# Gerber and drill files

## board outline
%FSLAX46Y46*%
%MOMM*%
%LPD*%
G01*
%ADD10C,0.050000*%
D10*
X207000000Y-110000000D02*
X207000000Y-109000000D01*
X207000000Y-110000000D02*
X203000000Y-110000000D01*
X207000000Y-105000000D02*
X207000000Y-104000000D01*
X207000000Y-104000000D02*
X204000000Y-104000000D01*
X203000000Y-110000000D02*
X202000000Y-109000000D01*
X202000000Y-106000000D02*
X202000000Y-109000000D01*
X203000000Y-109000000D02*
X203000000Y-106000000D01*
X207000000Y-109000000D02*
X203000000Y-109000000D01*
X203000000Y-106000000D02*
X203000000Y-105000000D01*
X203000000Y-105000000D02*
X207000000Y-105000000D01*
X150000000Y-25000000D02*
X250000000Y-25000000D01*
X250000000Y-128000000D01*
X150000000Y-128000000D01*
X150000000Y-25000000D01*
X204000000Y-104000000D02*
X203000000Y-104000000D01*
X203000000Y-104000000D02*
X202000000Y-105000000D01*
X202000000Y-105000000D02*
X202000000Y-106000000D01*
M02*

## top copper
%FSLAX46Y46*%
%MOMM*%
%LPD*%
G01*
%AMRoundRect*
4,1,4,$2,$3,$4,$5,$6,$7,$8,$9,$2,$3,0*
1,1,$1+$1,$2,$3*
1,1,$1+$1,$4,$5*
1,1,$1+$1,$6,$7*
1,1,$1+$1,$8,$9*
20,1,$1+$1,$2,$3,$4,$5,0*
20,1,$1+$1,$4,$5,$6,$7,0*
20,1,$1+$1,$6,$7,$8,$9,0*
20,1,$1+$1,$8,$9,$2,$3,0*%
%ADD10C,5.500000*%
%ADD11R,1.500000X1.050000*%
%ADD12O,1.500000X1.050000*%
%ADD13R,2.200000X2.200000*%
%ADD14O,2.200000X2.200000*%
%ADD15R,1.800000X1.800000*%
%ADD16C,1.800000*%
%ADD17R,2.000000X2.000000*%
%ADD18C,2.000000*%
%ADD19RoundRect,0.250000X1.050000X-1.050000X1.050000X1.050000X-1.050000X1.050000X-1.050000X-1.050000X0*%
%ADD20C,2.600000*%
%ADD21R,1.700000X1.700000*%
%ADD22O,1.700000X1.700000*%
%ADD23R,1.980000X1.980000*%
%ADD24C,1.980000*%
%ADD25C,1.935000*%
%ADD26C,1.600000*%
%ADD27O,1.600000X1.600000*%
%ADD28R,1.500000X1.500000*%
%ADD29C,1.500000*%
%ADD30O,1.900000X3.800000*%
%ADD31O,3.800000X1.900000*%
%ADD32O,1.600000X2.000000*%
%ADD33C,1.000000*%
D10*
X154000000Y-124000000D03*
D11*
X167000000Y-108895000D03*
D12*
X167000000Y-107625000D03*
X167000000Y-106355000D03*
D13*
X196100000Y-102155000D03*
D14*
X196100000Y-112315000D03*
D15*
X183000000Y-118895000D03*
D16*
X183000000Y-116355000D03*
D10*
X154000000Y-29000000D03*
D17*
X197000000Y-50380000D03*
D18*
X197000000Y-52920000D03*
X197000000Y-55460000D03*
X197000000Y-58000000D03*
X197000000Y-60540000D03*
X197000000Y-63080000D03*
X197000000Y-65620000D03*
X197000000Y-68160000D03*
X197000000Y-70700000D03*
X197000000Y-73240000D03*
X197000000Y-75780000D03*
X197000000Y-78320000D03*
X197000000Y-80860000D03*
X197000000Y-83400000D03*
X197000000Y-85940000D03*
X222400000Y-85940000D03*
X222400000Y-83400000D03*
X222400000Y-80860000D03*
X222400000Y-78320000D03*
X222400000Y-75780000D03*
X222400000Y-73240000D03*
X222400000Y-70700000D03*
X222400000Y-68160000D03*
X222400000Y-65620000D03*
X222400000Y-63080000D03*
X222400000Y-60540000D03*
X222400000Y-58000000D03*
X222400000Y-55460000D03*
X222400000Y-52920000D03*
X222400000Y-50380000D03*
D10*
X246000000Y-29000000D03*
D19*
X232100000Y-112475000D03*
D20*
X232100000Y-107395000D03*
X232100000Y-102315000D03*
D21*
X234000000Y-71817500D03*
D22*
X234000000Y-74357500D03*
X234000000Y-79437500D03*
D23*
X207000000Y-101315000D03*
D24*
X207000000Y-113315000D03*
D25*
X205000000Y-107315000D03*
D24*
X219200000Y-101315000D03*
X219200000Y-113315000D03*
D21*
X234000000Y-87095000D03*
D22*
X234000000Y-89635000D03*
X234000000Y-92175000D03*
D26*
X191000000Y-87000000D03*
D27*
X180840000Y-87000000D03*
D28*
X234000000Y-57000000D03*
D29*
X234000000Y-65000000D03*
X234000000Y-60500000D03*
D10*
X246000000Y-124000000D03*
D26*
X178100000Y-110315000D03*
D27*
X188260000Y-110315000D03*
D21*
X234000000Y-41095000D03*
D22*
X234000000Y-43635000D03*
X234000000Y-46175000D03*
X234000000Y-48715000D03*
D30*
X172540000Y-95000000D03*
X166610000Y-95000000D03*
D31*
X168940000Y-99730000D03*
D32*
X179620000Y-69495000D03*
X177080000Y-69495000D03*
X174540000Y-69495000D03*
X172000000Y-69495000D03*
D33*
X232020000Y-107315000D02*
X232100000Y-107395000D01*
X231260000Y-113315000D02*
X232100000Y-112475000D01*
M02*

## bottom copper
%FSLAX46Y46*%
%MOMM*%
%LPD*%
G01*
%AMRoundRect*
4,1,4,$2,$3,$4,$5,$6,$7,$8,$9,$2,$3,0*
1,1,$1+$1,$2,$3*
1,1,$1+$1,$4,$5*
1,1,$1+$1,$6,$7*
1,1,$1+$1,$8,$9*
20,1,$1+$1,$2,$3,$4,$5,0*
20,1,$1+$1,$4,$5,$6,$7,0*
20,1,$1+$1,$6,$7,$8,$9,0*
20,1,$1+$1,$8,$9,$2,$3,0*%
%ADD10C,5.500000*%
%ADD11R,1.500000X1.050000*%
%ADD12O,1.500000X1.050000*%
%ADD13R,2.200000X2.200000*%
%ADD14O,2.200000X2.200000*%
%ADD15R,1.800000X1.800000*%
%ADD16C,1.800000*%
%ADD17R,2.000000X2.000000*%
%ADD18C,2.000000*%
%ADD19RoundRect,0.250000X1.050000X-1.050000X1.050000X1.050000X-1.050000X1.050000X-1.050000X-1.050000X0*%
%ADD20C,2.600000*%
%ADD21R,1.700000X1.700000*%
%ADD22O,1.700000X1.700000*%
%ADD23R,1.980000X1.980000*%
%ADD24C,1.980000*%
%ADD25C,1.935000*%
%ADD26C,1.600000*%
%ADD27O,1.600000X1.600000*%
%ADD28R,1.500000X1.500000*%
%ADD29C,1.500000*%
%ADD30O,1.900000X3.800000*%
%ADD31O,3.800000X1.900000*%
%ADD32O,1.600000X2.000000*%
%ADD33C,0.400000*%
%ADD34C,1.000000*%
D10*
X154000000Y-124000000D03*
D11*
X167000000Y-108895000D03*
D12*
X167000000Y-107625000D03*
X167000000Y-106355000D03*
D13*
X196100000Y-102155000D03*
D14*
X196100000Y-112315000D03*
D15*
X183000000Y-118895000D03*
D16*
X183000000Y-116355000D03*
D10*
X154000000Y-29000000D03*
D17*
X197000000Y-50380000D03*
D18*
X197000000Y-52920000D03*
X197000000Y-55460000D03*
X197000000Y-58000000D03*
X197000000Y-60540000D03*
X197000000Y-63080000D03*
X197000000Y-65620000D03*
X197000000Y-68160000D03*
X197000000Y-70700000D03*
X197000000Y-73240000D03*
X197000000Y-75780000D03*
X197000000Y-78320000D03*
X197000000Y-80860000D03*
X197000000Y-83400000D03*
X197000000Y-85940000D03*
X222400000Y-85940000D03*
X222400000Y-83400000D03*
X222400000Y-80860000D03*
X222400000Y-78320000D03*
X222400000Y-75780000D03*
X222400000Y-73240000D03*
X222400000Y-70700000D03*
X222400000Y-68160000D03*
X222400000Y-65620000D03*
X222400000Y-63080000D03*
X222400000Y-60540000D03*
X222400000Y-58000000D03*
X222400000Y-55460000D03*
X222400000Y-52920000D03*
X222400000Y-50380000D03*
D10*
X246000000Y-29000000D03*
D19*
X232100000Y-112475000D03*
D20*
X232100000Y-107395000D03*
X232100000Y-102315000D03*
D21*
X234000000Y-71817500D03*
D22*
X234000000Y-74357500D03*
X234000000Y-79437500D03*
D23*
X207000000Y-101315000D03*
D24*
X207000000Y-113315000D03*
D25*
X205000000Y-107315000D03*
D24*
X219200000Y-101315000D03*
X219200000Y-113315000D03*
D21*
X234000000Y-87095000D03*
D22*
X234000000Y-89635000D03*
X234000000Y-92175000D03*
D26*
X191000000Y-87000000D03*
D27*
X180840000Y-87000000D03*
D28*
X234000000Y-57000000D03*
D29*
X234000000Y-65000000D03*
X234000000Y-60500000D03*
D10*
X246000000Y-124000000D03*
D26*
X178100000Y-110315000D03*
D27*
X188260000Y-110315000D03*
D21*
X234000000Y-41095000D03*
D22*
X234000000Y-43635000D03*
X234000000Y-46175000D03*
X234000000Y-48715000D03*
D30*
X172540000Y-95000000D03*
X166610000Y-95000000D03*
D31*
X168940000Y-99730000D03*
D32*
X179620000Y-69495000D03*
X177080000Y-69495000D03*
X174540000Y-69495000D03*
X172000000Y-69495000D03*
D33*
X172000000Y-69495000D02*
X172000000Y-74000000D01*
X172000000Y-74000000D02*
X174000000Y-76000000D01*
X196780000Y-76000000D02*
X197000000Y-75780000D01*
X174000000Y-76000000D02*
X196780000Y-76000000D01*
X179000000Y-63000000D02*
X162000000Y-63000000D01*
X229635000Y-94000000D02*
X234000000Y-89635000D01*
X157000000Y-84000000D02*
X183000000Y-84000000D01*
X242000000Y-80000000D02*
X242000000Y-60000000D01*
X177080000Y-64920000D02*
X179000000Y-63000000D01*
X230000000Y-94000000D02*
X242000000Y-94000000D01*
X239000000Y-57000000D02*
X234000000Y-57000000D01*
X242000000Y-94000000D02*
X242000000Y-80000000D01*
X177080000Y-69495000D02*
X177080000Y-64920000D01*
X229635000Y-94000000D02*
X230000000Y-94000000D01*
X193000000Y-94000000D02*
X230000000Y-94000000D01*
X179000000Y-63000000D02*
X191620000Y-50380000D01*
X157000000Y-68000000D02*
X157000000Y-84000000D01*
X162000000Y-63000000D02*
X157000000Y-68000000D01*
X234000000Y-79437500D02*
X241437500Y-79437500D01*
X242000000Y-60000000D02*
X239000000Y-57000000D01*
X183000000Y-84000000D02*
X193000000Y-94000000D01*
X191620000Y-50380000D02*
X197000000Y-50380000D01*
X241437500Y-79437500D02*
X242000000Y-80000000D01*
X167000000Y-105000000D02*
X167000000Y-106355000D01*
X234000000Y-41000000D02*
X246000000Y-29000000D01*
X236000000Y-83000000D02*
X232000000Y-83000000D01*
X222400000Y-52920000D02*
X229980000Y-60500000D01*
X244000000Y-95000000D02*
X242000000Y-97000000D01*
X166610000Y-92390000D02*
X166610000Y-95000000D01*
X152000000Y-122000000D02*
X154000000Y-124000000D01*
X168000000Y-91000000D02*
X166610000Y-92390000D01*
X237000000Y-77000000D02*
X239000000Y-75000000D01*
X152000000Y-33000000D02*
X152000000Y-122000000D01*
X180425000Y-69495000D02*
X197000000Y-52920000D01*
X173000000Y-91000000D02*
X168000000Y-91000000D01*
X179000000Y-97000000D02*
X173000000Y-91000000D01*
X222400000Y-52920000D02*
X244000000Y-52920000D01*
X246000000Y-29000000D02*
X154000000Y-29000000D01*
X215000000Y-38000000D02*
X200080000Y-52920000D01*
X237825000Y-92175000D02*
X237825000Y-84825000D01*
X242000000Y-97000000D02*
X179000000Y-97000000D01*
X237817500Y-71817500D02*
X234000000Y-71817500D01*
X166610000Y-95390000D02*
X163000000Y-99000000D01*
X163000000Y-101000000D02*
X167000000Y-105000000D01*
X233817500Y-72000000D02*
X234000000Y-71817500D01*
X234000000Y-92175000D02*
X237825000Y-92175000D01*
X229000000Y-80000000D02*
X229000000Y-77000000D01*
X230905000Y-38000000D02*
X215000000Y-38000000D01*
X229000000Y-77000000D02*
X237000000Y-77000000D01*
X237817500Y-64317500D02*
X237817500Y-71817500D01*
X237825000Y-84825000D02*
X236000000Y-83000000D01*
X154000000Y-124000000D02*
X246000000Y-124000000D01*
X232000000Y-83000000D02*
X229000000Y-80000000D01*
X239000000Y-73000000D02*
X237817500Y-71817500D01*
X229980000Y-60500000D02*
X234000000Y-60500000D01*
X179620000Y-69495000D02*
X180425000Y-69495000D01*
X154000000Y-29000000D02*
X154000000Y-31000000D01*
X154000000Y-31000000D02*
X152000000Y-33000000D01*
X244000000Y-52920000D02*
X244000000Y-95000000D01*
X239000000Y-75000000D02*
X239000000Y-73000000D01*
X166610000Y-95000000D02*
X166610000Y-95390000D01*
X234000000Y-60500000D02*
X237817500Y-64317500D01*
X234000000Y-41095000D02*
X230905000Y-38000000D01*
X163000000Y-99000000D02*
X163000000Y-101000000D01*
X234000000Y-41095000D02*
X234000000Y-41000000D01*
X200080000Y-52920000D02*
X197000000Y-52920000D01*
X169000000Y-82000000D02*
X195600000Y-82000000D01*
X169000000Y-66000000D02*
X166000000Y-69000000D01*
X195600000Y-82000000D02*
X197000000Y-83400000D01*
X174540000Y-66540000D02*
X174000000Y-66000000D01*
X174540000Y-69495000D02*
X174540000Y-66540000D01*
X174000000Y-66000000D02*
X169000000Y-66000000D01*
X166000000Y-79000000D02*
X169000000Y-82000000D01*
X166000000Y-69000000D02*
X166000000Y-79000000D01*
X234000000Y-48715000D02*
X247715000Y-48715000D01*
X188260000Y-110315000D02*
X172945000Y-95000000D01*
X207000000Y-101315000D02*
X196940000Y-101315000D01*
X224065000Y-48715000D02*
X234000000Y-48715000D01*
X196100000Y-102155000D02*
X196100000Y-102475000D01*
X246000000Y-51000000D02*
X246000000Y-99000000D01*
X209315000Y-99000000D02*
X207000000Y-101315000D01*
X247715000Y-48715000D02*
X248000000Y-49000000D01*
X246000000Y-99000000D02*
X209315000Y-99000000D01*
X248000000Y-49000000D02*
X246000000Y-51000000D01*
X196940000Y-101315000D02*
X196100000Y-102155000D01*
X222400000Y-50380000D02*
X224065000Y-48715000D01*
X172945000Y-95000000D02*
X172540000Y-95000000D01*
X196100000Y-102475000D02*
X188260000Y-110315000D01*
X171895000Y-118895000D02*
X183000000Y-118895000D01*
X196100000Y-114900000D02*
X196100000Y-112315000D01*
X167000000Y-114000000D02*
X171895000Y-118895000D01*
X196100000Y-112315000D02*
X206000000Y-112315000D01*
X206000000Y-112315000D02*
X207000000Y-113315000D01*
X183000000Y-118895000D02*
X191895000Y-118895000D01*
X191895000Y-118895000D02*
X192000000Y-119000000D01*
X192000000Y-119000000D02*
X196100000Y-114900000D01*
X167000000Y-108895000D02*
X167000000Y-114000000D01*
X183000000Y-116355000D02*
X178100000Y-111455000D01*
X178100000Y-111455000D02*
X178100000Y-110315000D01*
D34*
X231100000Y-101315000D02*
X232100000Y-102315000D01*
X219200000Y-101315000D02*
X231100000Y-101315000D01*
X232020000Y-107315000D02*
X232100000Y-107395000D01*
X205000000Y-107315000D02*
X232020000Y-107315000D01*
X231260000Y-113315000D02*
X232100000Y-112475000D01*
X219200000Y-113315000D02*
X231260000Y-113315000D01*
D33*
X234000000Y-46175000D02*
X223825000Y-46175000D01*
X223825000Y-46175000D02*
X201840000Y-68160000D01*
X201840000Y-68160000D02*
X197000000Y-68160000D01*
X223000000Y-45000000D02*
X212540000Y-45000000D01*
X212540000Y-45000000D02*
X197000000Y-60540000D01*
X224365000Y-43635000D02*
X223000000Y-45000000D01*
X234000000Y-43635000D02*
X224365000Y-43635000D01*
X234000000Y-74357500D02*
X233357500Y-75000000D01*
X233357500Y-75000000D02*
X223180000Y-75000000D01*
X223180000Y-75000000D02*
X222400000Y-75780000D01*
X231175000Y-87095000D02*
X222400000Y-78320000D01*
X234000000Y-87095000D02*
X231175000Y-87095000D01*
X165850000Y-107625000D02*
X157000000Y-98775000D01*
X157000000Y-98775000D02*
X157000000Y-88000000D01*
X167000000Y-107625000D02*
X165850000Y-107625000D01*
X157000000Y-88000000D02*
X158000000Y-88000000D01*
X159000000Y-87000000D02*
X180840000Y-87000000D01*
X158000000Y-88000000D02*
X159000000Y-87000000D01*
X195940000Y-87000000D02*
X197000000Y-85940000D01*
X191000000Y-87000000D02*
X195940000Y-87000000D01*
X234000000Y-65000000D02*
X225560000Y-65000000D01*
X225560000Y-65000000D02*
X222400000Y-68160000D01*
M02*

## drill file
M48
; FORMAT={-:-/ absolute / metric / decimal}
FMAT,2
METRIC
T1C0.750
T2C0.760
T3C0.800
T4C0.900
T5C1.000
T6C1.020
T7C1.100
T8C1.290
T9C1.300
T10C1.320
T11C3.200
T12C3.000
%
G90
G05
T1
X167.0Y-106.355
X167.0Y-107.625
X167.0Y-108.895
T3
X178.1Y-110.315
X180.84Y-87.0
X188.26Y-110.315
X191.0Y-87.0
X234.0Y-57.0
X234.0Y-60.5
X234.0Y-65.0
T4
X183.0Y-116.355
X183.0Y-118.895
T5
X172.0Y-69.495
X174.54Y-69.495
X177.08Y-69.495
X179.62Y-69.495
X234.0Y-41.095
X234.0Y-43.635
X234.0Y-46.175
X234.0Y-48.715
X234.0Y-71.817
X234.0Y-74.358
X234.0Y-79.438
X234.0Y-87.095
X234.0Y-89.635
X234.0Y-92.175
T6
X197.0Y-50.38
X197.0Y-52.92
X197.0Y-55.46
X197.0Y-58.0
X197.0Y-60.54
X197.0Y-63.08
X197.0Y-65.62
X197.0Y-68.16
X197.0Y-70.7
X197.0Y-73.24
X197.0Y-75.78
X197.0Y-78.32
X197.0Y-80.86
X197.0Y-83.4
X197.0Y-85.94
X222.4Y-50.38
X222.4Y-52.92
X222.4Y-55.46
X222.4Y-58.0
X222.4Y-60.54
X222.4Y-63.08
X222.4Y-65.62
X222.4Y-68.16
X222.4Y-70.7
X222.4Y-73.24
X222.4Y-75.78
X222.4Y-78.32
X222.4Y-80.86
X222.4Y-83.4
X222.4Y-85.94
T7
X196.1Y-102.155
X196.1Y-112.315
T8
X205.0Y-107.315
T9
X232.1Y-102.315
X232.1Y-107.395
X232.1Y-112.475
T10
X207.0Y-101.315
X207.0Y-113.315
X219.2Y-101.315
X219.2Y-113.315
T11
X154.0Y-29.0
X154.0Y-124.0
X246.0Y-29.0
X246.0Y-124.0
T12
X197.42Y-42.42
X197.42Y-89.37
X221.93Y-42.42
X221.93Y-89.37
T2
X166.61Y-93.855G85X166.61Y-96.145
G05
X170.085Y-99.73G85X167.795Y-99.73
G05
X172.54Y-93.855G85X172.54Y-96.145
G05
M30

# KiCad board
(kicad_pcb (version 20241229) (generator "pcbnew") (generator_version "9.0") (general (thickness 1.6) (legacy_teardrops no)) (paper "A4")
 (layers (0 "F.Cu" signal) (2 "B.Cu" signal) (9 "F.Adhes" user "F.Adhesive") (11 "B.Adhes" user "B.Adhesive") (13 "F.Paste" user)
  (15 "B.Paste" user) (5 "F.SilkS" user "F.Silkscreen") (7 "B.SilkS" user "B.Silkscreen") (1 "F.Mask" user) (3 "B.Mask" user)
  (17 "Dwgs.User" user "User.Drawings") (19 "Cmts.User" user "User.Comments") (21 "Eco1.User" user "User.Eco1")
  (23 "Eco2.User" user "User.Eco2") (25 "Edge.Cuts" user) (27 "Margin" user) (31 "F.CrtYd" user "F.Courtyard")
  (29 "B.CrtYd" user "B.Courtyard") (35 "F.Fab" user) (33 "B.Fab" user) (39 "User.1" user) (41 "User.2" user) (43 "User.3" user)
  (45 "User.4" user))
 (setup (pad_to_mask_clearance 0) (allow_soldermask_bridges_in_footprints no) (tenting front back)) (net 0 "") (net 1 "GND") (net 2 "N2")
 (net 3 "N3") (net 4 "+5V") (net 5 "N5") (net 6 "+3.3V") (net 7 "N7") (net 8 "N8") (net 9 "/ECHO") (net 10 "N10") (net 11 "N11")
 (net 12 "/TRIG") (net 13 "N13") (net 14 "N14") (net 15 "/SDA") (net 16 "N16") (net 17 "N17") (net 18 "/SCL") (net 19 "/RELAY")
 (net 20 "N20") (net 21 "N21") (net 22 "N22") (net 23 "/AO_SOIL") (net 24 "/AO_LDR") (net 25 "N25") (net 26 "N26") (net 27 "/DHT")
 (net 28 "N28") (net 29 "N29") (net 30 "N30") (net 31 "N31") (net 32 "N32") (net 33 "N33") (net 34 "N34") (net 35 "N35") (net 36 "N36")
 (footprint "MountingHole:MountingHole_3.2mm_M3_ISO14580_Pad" (layer "F.Cu") (at 154 124)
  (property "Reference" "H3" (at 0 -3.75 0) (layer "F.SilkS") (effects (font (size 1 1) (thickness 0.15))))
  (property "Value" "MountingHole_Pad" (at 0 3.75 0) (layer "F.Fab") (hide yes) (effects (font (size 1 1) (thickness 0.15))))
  (pad "1" thru_hole circle (at 0 0) (size 5.5 5.5) (drill 3.2) (layers "*.Cu" "*.Mask") (remove_unused_layers no) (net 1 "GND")))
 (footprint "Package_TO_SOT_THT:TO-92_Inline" (layer "F.Cu") (at 167 108.895 90)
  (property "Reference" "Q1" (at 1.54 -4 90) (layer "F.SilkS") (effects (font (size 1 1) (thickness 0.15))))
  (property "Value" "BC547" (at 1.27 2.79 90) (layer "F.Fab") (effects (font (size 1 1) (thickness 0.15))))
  (pad "1" thru_hole rect (at 0 0 90) (size 1.05 1.5) (drill 0.75) (layers "*.Cu" "*.Mask") (remove_unused_layers no) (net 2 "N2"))
  (pad "2" thru_hole oval (at 1.27 0 90) (size 1.05 1.5) (drill 0.75) (layers "*.Cu" "*.Mask") (remove_unused_layers no) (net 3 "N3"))
  (pad "3" thru_hole oval (at 2.54 0 90) (size 1.05 1.5) (drill 0.75) (layers "*.Cu" "*.Mask") (remove_unused_layers no) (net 1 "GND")))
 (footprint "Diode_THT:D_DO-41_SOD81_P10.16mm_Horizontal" (layer "F.Cu") (at 196.1 102.155 -90)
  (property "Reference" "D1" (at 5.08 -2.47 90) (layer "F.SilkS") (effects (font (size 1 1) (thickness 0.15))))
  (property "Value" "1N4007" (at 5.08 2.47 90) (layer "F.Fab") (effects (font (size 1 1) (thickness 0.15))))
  (pad "1" thru_hole rect (at 0 0 270) (size 2.2 2.2) (drill 1.1) (layers "*.Cu" "*.Mask") (remove_unused_layers no) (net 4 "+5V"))
  (pad "2" thru_hole oval (at 10.16 0 270) (size 2.2 2.2) (drill 1.1) (layers "*.Cu" "*.Mask") (remove_unused_layers no) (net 2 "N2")))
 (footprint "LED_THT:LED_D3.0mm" (layer "F.Cu") (at 183 118.895 90)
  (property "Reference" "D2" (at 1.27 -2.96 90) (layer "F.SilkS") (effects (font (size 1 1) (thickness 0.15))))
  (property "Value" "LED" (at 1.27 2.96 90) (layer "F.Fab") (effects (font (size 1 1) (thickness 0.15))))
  (pad "1" thru_hole rect (at 0 0 90) (size 1.8 1.8) (drill 0.9) (layers "*.Cu" "*.Mask") (remove_unused_layers no) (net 2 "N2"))
  (pad "2" thru_hole circle (at 2.54 0 90) (size 1.8 1.8) (drill 0.9) (layers "*.Cu" "*.Mask") (remove_unused_layers no) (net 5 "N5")))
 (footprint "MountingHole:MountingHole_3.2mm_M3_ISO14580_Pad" (layer "F.Cu") (at 154 29)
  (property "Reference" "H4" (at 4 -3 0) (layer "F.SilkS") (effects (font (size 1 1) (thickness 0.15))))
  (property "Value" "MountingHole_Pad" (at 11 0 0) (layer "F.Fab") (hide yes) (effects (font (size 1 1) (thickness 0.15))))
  (pad "1" thru_hole circle (at 0 0) (size 5.5 5.5) (drill 3.2) (layers "*.Cu" "*.Mask") (remove_unused_layers no) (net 1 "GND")))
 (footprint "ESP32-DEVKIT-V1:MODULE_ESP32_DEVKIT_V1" (layer "F.Cu") (at 209.7 65.895)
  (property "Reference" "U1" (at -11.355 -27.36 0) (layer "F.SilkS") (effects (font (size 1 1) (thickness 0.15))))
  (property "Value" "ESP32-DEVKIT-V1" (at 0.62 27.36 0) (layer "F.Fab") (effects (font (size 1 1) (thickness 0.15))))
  (pad "" np_thru_hole circle (at -12.28 -23.475) (size 3 3) (drill 3) (layers "*.Cu" "*.Mask"))
  (pad "" np_thru_hole circle (at -12.28 23.475) (size 3 3) (drill 3) (layers "*.Cu" "*.Mask"))
  (pad "" np_thru_hole circle (at 12.23 -23.475) (size 3 3) (drill 3) (layers "*.Cu" "*.Mask"))
  (pad "" np_thru_hole circle (at 12.23 23.475) (size 3 3) (drill 3) (layers "*.Cu" "*.Mask"))
  (pad "1" thru_hole rect (at -12.7 -15.515) (size 2 2) (drill 1.02) (layers "*.Cu" "*.Mask") (remove_unused_layers no) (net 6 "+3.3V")
   (solder_mask_margin 0.102))
  (pad "2" thru_hole circle (at -12.7 -12.975) (size 2 2) (drill 1.02) (layers "*.Cu" "*.Mask") (remove_unused_layers no) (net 1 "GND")
   (solder_mask_margin 0.102))
  (pad "3" thru_hole circle (at -12.7 -10.435) (size 2 2) (drill 1.02) (layers "*.Cu" "*.Mask") (remove_unused_layers no) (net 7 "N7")
   (solder_mask_margin 0.102))
  (pad "4" thru_hole circle (at -12.7 -7.895) (size 2 2) (drill 1.02) (layers "*.Cu" "*.Mask") (remove_unused_layers no) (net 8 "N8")
   (solder_mask_margin 0.102))
  (pad "5" thru_hole circle (at -12.7 -5.355) (size 2 2) (drill 1.02) (layers "*.Cu" "*.Mask") (remove_unused_layers no) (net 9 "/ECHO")
   (solder_mask_margin 0.102))
  (pad "6" thru_hole circle (at -12.7 -2.815) (size 2 2) (drill 1.02) (layers "*.Cu" "*.Mask") (remove_unused_layers no) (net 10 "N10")
   (solder_mask_margin 0.102))
  (pad "7" thru_hole circle (at -12.7 -0.275) (size 2 2) (drill 1.02) (layers "*.Cu" "*.Mask") (remove_unused_layers no) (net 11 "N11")
   (solder_mask_margin 0.102))
  (pad "8" thru_hole circle (at -12.7 2.265) (size 2 2) (drill 1.02) (layers "*.Cu" "*.Mask") (remove_unused_layers no) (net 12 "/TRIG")
   (solder_mask_margin 0.102))
  (pad "9" thru_hole circle (at -12.7 4.805) (size 2 2) (drill 1.02) (layers "*.Cu" "*.Mask") (remove_unused_layers no) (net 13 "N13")
   (solder_mask_margin 0.102))
  (pad "10" thru_hole circle (at -12.7 7.345) (size 2 2) (drill 1.02) (layers "*.Cu" "*.Mask") (remove_unused_layers no) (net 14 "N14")
   (solder_mask_margin 0.102))
  (pad "11" thru_hole circle (at -12.7 9.885) (size 2 2) (drill 1.02) (layers "*.Cu" "*.Mask") (remove_unused_layers no) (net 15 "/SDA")
   (solder_mask_margin 0.102))
  (pad "12" thru_hole circle (at -12.7 12.425) (size 2 2) (drill 1.02) (layers "*.Cu" "*.Mask") (remove_unused_layers no) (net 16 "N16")
   (solder_mask_margin 0.102))
  (pad "13" thru_hole circle (at -12.7 14.965) (size 2 2) (drill 1.02) (layers "*.Cu" "*.Mask") (remove_unused_layers no) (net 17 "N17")
   (solder_mask_margin 0.102))
  (pad "14" thru_hole circle (at -12.7 17.505) (size 2 2) (drill 1.02) (layers "*.Cu" "*.Mask") (remove_unused_layers no) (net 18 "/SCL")
   (solder_mask_margin 0.102))
  (pad "15" thru_hole circle (at -12.7 20.045) (size 2 2) (drill 1.02) (layers "*.Cu" "*.Mask") (remove_unused_layers no) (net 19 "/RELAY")
   (solder_mask_margin 0.102))
  (pad "16" thru_hole circle (at 12.7 20.045) (size 2 2) (drill 1.02) (layers "*.Cu" "*.Mask") (remove_unused_layers no) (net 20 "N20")
   (solder_mask_margin 0.102))
  (pad "17" thru_hole circle (at 12.7 17.505) (size 2 2) (drill 1.02) (layers "*.Cu" "*.Mask") (remove_unused_layers no) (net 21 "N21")
   (solder_mask_margin 0.102))
  (pad "18" thru_hole circle (at 12.7 14.965) (size 2 2) (drill 1.02) (layers "*.Cu" "*.Mask") (remove_unused_layers no) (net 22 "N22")
   (solder_mask_margin 0.102))
  (pad "19" thru_hole circle (at 12.7 12.425) (size 2 2) (drill 1.02) (layers "*.Cu" "*.Mask") (remove_unused_layers no) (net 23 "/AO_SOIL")
   (solder_mask_margin 0.102))
  (pad "20" thru_hole circle (at 12.7 9.885) (size 2 2) (drill 1.02) (layers "*.Cu" "*.Mask") (remove_unused_layers no) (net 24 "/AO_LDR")
   (solder_mask_margin 0.102))
  (pad "21" thru_hole circle (at 12.7 7.345) (size 2 2) (drill 1.02) (layers "*.Cu" "*.Mask") (remove_unused_layers no) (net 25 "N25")
   (solder_mask_margin 0.102))
  (pad "22" thru_hole circle (at 12.7 4.805) (size 2 2) (drill 1.02) (layers "*.Cu" "*.Mask") (remove_unused_layers no) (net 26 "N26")
   (solder_mask_margin 0.102))
  (pad "23" thru_hole circle (at 12.7 2.265) (size 2 2) (drill 1.02) (layers "*.Cu" "*.Mask") (remove_unused_layers no) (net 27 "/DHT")
   (solder_mask_margin 0.102))
  (pad "24" thru_hole circle (at 12.7 -0.275) (size 2 2) (drill 1.02) (layers "*.Cu" "*.Mask") (remove_unused_layers no) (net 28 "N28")
   (solder_mask_margin 0.102))
  (pad "25" thru_hole circle (at 12.7 -2.815) (size 2 2) (drill 1.02) (layers "*.Cu" "*.Mask") (remove_unused_layers no) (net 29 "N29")
   (solder_mask_margin 0.102))
  (pad "26" thru_hole circle (at 12.7 -5.355) (size 2 2) (drill 1.02) (layers "*.Cu" "*.Mask") (remove_unused_layers no) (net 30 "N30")
   (solder_mask_margin 0.102))
  (pad "27" thru_hole circle (at 12.7 -7.895) (size 2 2) (drill 1.02) (layers "*.Cu" "*.Mask") (remove_unused_layers no) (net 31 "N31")
   (solder_mask_margin 0.102))
  (pad "28" thru_hole circle (at 12.7 -10.435) (size 2 2) (drill 1.02) (layers "*.Cu" "*.Mask") (remove_unused_layers no) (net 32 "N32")
   (solder_mask_margin 0.102))
  (pad "29" thru_hole circle (at 12.7 -12.975) (size 2 2) (drill 1.02) (layers "*.Cu" "*.Mask") (remove_unused_layers no) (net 1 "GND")
   (solder_mask_margin 0.102))
  (pad "30" thru_hole circle (at 12.7 -15.515) (size 2 2) (drill 1.02) (layers "*.Cu" "*.Mask") (remove_unused_layers no) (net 4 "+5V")
   (solder_mask_margin 0.102))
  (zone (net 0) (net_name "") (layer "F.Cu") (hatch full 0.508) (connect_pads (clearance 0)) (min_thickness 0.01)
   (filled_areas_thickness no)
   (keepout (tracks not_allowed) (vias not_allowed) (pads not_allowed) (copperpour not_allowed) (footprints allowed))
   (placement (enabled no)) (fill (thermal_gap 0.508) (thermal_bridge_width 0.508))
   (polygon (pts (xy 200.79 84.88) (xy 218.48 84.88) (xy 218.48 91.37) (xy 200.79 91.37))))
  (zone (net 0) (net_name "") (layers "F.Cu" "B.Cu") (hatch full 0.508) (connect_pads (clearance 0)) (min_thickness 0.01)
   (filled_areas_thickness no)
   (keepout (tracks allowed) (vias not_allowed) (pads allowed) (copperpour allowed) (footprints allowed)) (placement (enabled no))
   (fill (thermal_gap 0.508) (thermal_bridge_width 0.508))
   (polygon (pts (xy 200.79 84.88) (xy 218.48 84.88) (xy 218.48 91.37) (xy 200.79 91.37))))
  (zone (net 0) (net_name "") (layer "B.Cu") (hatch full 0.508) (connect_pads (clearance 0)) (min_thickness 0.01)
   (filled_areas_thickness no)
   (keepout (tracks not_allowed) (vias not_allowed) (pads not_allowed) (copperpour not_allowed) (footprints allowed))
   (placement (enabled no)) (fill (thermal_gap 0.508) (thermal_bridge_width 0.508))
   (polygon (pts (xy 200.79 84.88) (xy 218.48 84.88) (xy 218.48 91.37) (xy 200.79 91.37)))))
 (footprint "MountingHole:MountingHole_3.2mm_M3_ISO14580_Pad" (layer "F.Cu") (at 246 29)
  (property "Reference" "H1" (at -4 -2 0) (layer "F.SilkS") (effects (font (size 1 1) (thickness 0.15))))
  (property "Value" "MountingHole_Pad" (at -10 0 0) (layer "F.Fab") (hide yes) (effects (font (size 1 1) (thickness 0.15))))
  (pad "1" thru_hole circle (at 0 0) (size 5.5 5.5) (drill 3.2) (layers "*.Cu" "*.Mask") (remove_unused_layers no) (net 1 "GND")))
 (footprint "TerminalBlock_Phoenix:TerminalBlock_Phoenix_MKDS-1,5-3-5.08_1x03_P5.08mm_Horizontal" (layer "F.Cu") (at 232.1 112.475 90)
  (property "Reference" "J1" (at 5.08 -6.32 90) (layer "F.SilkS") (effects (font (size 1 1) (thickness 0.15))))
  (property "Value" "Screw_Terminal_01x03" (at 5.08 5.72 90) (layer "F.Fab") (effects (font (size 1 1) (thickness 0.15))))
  (pad "1" thru_hole roundrect (at 0 0 90) (size 2.6 2.6) (drill 1.3) (layers "*.Cu" "*.Mask") (remove_unused_layers no)
   (roundrect_rratio 0.096154) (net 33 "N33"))
  (pad "2" thru_hole circle (at 5.08 0 90) (size 2.6 2.6) (drill 1.3) (layers "*.Cu" "*.Mask") (remove_unused_layers no) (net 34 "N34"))
  (pad "3" thru_hole circle (at 10.16 0 90) (size 2.6 2.6) (drill 1.3) (layers "*.Cu" "*.Mask") (remove_unused_layers no) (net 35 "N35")))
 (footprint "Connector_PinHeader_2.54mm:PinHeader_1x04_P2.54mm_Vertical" (layer "F.Cu") (at 234 71.8175)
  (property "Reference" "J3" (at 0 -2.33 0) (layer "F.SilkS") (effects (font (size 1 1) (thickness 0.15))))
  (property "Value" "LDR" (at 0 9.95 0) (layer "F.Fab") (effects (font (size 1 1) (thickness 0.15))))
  (pad "1" thru_hole rect (at 0 0) (size 1.7 1.7) (drill 1) (layers "*.Cu" "*.Mask") (remove_unused_layers no) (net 1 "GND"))
  (pad "2" thru_hole oval (at 0 2.54) (size 1.7 1.7) (drill 1) (layers "*.Cu" "*.Mask") (remove_unused_layers no) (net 24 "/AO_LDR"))
  (pad "4" thru_hole oval (at 0 7.62) (size 1.7 1.7) (drill 1) (layers "*.Cu" "*.Mask") (remove_unused_layers no) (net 6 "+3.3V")))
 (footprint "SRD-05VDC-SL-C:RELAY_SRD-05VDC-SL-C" (layer "F.Cu") (at 213.1 107.315)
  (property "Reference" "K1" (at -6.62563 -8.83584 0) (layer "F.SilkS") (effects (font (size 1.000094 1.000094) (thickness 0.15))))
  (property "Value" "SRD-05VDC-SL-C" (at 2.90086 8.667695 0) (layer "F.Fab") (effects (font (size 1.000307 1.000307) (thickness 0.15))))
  (pad "A1" thru_hole rect (at -6.1 -6) (size 1.98 1.98) (drill 1.32) (layers "*.Cu" "*.Mask") (remove_unused_layers no) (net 4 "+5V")
   (solder_mask_margin 0.102))
  (pad "A2" thru_hole circle (at -6.1 6) (size 1.98 1.98) (drill 1.32) (layers "*.Cu" "*.Mask") (remove_unused_layers no) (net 2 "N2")
   (solder_mask_margin 0.102))
  (pad "COM" thru_hole circle (at -8.1 0) (size 1.935 1.935) (drill 1.29) (layers "*.Cu" "*.Mask") (remove_unused_layers no) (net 34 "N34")
   (solder_mask_margin 0.102))
  (pad "NC" thru_hole circle (at 6.1 -6) (size 1.98 1.98) (drill 1.32) (layers "*.Cu" "*.Mask") (remove_unused_layers no) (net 35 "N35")
   (solder_mask_margin 0.102))
  (pad "NO" thru_hole circle (at 6.1 6) (size 1.98 1.98) (drill 1.32) (layers "*.Cu" "*.Mask") (remove_unused_layers no) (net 33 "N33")
   (solder_mask_margin 0.102)))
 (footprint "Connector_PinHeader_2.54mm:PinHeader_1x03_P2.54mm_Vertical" (layer "F.Cu") (at 234 87.095)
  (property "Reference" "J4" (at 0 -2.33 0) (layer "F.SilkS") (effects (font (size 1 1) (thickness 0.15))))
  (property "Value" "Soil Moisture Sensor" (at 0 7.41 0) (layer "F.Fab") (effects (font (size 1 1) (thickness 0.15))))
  (pad "1" thru_hole rect (at 0 0) (size 1.7 1.7) (drill 1) (layers "*.Cu" "*.Mask") (remove_unused_layers no) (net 23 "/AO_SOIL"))
  (pad "2" thru_hole oval (at 0 2.54) (size 1.7 1.7) (drill 1) (layers "*.Cu" "*.Mask") (remove_unused_layers no) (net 6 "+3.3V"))
  (pad "3" thru_hole oval (at 0 5.08) (size 1.7 1.7) (drill 1) (layers "*.Cu" "*.Mask") (remove_unused_layers no) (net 1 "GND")))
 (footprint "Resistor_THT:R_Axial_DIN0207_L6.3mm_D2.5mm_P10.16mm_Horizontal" (layer "F.Cu") (at 191 87 180)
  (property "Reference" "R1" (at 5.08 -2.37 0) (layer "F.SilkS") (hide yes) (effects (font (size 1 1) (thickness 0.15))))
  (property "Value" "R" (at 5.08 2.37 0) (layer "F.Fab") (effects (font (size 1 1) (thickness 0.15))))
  (pad "1" thru_hole circle (at 0 0 180) (size 1.6 1.6) (drill 0.8) (layers "*.Cu" "*.Mask") (remove_unused_layers no) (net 19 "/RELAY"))
  (pad "2" thru_hole oval (at 10.16 0 180) (size 1.6 1.6) (drill 0.8) (layers "*.Cu" "*.Mask") (remove_unused_layers no) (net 3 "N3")))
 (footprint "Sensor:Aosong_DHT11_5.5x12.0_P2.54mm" (layer "F.Cu") (at 234 57)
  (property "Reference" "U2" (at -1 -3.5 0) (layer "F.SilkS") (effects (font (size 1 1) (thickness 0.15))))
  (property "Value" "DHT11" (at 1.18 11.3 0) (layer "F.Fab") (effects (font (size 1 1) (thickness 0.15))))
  (pad "1" thru_hole rect (at 0 0) (size 1.5 1.5) (drill 0.8) (layers "*.Cu" "*.Mask") (remove_unused_layers no) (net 6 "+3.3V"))
  (pad "2" thru_hole circle (at 0 8) (size 1.5 1.5) (drill 0.8) (layers "*.Cu" "*.Mask") (remove_unused_layers no) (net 27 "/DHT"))
  (pad "4" thru_hole circle (at 0 3.5) (size 1.5 1.5) (drill 0.8) (layers "*.Cu" "*.Mask") (remove_unused_layers no) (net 1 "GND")))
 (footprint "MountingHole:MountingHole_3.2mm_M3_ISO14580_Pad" (layer "F.Cu") (at 246 124)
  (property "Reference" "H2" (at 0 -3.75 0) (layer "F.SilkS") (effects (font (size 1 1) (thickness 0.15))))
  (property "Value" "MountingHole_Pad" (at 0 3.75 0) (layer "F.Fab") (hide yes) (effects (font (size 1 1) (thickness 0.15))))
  (pad "1" thru_hole circle (at 0 0) (size 5.5 5.5) (drill 3.2) (layers "*.Cu" "*.Mask") (remove_unused_layers no) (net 1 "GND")))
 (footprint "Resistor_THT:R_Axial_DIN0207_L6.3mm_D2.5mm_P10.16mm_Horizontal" (layer "F.Cu") (at 178.1 110.315)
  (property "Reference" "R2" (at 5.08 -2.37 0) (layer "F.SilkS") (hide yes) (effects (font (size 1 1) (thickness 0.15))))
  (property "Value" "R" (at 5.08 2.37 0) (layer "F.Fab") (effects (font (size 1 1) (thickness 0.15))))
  (pad "1" thru_hole circle (at 0 0) (size 1.6 1.6) (drill 0.8) (layers "*.Cu" "*.Mask") (remove_unused_layers no) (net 5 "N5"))
  (pad "2" thru_hole oval (at 10.16 0) (size 1.6 1.6) (drill 0.8) (layers "*.Cu" "*.Mask") (remove_unused_layers no) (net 4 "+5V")))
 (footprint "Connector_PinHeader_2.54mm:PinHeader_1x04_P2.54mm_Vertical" (layer "F.Cu") (at 234 41.095)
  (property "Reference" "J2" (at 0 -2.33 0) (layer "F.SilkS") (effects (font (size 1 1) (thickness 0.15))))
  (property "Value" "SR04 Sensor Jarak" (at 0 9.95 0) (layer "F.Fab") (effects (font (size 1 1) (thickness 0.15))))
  (pad "1" thru_hole rect (at 0 0) (size 1.7 1.7) (drill 1) (layers "*.Cu" "*.Mask") (remove_unused_layers no) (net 1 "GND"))
  (pad "2" thru_hole oval (at 0 2.54) (size 1.7 1.7) (drill 1) (layers "*.Cu" "*.Mask") (remove_unused_layers no) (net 9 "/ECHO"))
  (pad "3" thru_hole oval (at 0 5.08) (size 1.7 1.7) (drill 1) (layers "*.Cu" "*.Mask") (remove_unused_layers no) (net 12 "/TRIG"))
  (pad "4" thru_hole oval (at 0 7.62) (size 1.7 1.7) (drill 1) (layers "*.Cu" "*.Mask") (remove_unused_layers no) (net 4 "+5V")))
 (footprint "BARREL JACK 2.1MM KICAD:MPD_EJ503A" (layer "F.Cu") (at 166 95 -90)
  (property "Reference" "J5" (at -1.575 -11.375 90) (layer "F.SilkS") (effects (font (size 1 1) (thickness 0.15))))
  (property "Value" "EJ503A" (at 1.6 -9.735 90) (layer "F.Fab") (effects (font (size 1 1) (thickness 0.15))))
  (pad "1" thru_hole oval (at 0 -6.54 270) (size 3.8 1.9) (drill oval 3.05 0.76) (layers "*.Cu" "*.Mask") (remove_unused_layers no)
   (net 4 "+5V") (solder_mask_margin 0.102))
  (pad "2" thru_hole oval (at 0 -0.61 270) (size 3.8 1.9) (drill oval 3.05 0.76) (layers "*.Cu" "*.Mask") (remove_unused_layers no)
   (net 1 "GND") (solder_mask_margin 0.102))
  (pad "3" thru_hole oval (at 4.73 -2.94 270) (size 1.9 3.8) (drill oval 0.76 3.05) (layers "*.Cu" "*.Mask") (remove_unused_layers no)
   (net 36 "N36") (solder_mask_margin 0.102)))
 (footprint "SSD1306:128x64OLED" (layer "F.Cu") (at 176 58.895 180)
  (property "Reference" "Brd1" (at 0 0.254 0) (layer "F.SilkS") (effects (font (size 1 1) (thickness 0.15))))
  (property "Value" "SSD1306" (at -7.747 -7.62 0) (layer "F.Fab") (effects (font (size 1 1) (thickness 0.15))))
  (pad "1" thru_hole oval (at -3.62 -10.6 270) (size 2 1.6) (drill 1) (layers "*.Cu" "*.Mask") (remove_unused_layers no) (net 1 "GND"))
  (pad "2" thru_hole oval (at -1.08 -10.6 270) (size 2 1.6) (drill 1) (layers "*.Cu" "*.Mask") (remove_unused_layers no) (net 6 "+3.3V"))
  (pad "3" thru_hole oval (at 1.46 -10.6 270) (size 2 1.6) (drill 1) (layers "*.Cu" "*.Mask") (remove_unused_layers no) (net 18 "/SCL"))
  (pad "4" thru_hole oval (at 4 -10.6 270) (size 2 1.6) (drill 1) (layers "*.Cu" "*.Mask") (remove_unused_layers no) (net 15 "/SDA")))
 (gr_line (start 207 110) (end 207 109) (stroke (width 0.05) (type default)) (layer "Edge.Cuts"))
 (gr_line (start 207 110) (end 203 110) (stroke (width 0.05) (type default)) (layer "Edge.Cuts"))
 (gr_line (start 207 105) (end 207 104) (stroke (width 0.05) (type default)) (layer "Edge.Cuts"))
 (gr_line (start 207 104) (end 204 104) (stroke (width 0.05) (type default)) (layer "Edge.Cuts"))
 (gr_line (start 203 110) (end 202 109) (stroke (width 0.05) (type default)) (layer "Edge.Cuts"))
 (gr_line (start 202 106) (end 202 109) (stroke (width 0.05) (type default)) (layer "Edge.Cuts"))
 (gr_line (start 203 109) (end 203 106) (stroke (width 0.05) (type default)) (layer "Edge.Cuts"))
 (gr_line (start 207 109) (end 203 109) (stroke (width 0.05) (type default)) (layer "Edge.Cuts"))
 (gr_line (start 203 106) (end 203 105) (stroke (width 0.05) (type default)) (layer "Edge.Cuts"))
 (gr_line (start 203 105) (end 207 105) (stroke (width 0.05) (type default)) (layer "Edge.Cuts"))
 (gr_rect (start 150 25) (end 250 128) (stroke (width 0.05) (type default)) (fill no) (layer "Edge.Cuts"))
 (gr_line (start 204 104) (end 203 104) (stroke (width 0.05) (type default)) (layer "Edge.Cuts"))
 (gr_line (start 203 104) (end 202 105) (stroke (width 0.05) (type default)) (layer "Edge.Cuts"))
 (gr_line (start 202 105) (end 202 106) (stroke (width 0.05) (type default)) (layer "Edge.Cuts"))
 (segment (start 172 69.495) (end 172 74) (width 0.4) (layer "B.Cu") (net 15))
 (segment (start 172 74) (end 174 76) (width 0.4) (layer "B.Cu") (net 15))
 (segment (start 196.78 76) (end 197 75.78) (width 0.4) (layer "B.Cu") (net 15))
 (segment (start 174 76) (end 196.78 76) (width 0.4) (layer "B.Cu") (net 15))
 (segment (start 179 63) (end 162 63) (width 0.4) (layer "B.Cu") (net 6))
 (segment (start 229.635 94) (end 234 89.635) (width 0.4) (layer "B.Cu") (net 6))
 (segment (start 157 84) (end 183 84) (width 0.4) (layer "B.Cu") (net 6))
 (segment (start 242 80) (end 242 60) (width 0.4) (layer "B.Cu") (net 6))
 (segment (start 177.08 64.92) (end 179 63) (width 0.4) (layer "B.Cu") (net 6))
 (segment (start 230 94) (end 242 94) (width 0.4) (layer "B.Cu") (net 6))
 (segment (start 239 57) (end 234 57) (width 0.4) (layer "B.Cu") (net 6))
 (segment (start 242 94) (end 242 80) (width 0.4) (layer "B.Cu") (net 6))
 (segment (start 177.08 69.495) (end 177.08 64.92) (width 0.4) (layer "B.Cu") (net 6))
 (segment (start 229.635 94) (end 230 94) (width 0.4) (layer "B.Cu") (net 6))
 (segment (start 193 94) (end 230 94) (width 0.4) (layer "B.Cu") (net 6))
 (segment (start 179 63) (end 191.62 50.38) (width 0.4) (layer "B.Cu") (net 6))
 (segment (start 157 68) (end 157 84) (width 0.4) (layer "B.Cu") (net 6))
 (segment (start 162 63) (end 157 68) (width 0.4) (layer "B.Cu") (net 6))
 (segment (start 234 79.4375) (end 241.4375 79.4375) (width 0.4) (layer "B.Cu") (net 6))
 (segment (start 242 60) (end 239 57) (width 0.4) (layer "B.Cu") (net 6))
 (segment (start 183 84) (end 193 94) (width 0.4) (layer "B.Cu") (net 6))
 (segment (start 191.62 50.38) (end 197 50.38) (width 0.4) (layer "B.Cu") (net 6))
 (segment (start 241.4375 79.4375) (end 242 80) (width 0.4) (layer "B.Cu") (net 6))
 (segment (start 167 105) (end 167 106.355) (width 0.4) (layer "B.Cu") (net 1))
 (segment (start 234 41) (end 246 29) (width 0.4) (layer "B.Cu") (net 1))
 (segment (start 236 83) (end 232 83) (width 0.4) (layer "B.Cu") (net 1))
 (segment (start 222.4 52.92) (end 229.98 60.5) (width 0.4) (layer "B.Cu") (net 1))
 (segment (start 244 95) (end 242 97) (width 0.4) (layer "B.Cu") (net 1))
 (segment (start 166.61 92.39) (end 166.61 95) (width 0.4) (layer "B.Cu") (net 1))
 (segment (start 152 122) (end 154 124) (width 0.4) (layer "B.Cu") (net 1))
 (segment (start 168 91) (end 166.61 92.39) (width 0.4) (layer "B.Cu") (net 1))
 (segment (start 237 77) (end 239 75) (width 0.4) (layer "B.Cu") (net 1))
 (segment (start 152 33) (end 152 122) (width 0.4) (layer "B.Cu") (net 1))
 (segment (start 180.425 69.495) (end 197 52.92) (width 0.4) (layer "B.Cu") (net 1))
 (segment (start 173 91) (end 168 91) (width 0.4) (layer "B.Cu") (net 1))
 (segment (start 179 97) (end 173 91) (width 0.4) (layer "B.Cu") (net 1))
 (segment (start 222.4 52.92) (end 244 52.92) (width 0.4) (layer "B.Cu") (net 1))
 (segment (start 246 29) (end 154 29) (width 0.4) (layer "B.Cu") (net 1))
 (segment (start 215 38) (end 200.08 52.92) (width 0.4) (layer "B.Cu") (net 1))
 (segment (start 237.825 92.175) (end 237.825 84.825) (width 0.4) (layer "B.Cu") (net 1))
 (segment (start 242 97) (end 179 97) (width 0.4) (layer "B.Cu") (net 1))
 (segment (start 237.8175 71.8175) (end 234 71.8175) (width 0.4) (layer "B.Cu") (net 1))
 (segment (start 166.61 95.39) (end 163 99) (width 0.4) (layer "B.Cu") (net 1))
 (segment (start 163 101) (end 167 105) (width 0.4) (layer "B.Cu") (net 1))
 (segment (start 233.8175 72) (end 234 71.8175) (width 0.4) (layer "B.Cu") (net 1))
 (segment (start 234 92.175) (end 237.825 92.175) (width 0.4) (layer "B.Cu") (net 1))
 (segment (start 229 80) (end 229 77) (width 0.4) (layer "B.Cu") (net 1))
 (segment (start 230.905 38) (end 215 38) (width 0.4) (layer "B.Cu") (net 1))
 (segment (start 229 77) (end 237 77) (width 0.4) (layer "B.Cu") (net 1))
 (segment (start 237.8175 64.3175) (end 237.8175 71.8175) (width 0.4) (layer "B.Cu") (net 1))
 (segment (start 237.825 84.825) (end 236 83) (width 0.4) (layer "B.Cu") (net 1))
 (segment (start 154 124) (end 246 124) (width 0.4) (layer "B.Cu") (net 1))
 (segment (start 232 83) (end 229 80) (width 0.4) (layer "B.Cu") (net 1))
 (segment (start 239 73) (end 237.8175 71.8175) (width 0.4) (layer "B.Cu") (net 1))
 (segment (start 229.98 60.5) (end 234 60.5) (width 0.4) (layer "B.Cu") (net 1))
 (segment (start 179.62 69.495) (end 180.425 69.495) (width 0.4) (layer "B.Cu") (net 1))
 (segment (start 154 29) (end 154 31) (width 0.4) (layer "B.Cu") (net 1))
 (segment (start 154 31) (end 152 33) (width 0.4) (layer "B.Cu") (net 1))
 (segment (start 244 52.92) (end 244 95) (width 0.4) (layer "B.Cu") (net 1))
 (segment (start 239 75) (end 239 73) (width 0.4) (layer "B.Cu") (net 1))
 (segment (start 166.61 95) (end 166.61 95.39) (width 0.4) (layer "B.Cu") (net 1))
 (segment (start 234 60.5) (end 237.8175 64.3175) (width 0.4) (layer "B.Cu") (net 1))
 (segment (start 234 41.095) (end 230.905 38) (width 0.4) (layer "B.Cu") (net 1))
 (segment (start 163 99) (end 163 101) (width 0.4) (layer "B.Cu") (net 1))
 (segment (start 234 41.095) (end 234 41) (width 0.4) (layer "B.Cu") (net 1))
 (segment (start 200.08 52.92) (end 197 52.92) (width 0.4) (layer "B.Cu") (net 1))
 (segment (start 169 82) (end 195.6 82) (width 0.4) (layer "B.Cu") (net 18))
 (segment (start 169 66) (end 166 69) (width 0.4) (layer "B.Cu") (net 18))
 (segment (start 195.6 82) (end 197 83.4) (width 0.4) (layer "B.Cu") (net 18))
 (segment (start 174.54 66.54) (end 174 66) (width 0.4) (layer "B.Cu") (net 18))
 (segment (start 174.54 69.495) (end 174.54 66.54) (width 0.4) (layer "B.Cu") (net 18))
 (segment (start 174 66) (end 169 66) (width 0.4) (layer "B.Cu") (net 18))
 (segment (start 166 79) (end 169 82) (width 0.4) (layer "B.Cu") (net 18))
 (segment (start 166 69) (end 166 79) (width 0.4) (layer "B.Cu") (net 18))
 (segment (start 234 48.715) (end 247.715 48.715) (width 0.4) (layer "B.Cu") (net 4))
 (segment (start 188.26 110.315) (end 172.945 95) (width 0.4) (layer "B.Cu") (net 4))
 (segment (start 207 101.315) (end 196.94 101.315) (width 0.4) (layer "B.Cu") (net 4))
 (segment (start 224.065 48.715) (end 234 48.715) (width 0.4) (layer "B.Cu") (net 4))
 (segment (start 196.1 102.155) (end 196.1 102.475) (width 0.4) (layer "B.Cu") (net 4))
 (segment (start 246 51) (end 246 99) (width 0.4) (layer "B.Cu") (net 4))
 (segment (start 209.315 99) (end 207 101.315) (width 0.4) (layer "B.Cu") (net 4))
 (segment (start 247.715 48.715) (end 248 49) (width 0.4) (layer "B.Cu") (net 4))
 (segment (start 246 99) (end 209.315 99) (width 0.4) (layer "B.Cu") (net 4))
 (segment (start 248 49) (end 246 51) (width 0.4) (layer "B.Cu") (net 4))
 (segment (start 196.94 101.315) (end 196.1 102.155) (width 0.4) (layer "B.Cu") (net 4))
 (segment (start 222.4 50.38) (end 224.065 48.715) (width 0.4) (layer "B.Cu") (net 4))
 (segment (start 172.945 95) (end 172.54 95) (width 0.4) (layer "B.Cu") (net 4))
 (segment (start 196.1 102.475) (end 188.26 110.315) (width 0.4) (layer "B.Cu") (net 4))
 (segment (start 171.895 118.895) (end 183 118.895) (width 0.4) (layer "B.Cu") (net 2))
 (segment (start 196.1 114.9) (end 196.1 112.315) (width 0.4) (layer "B.Cu") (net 2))
 (segment (start 167 114) (end 171.895 118.895) (width 0.4) (layer "B.Cu") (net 2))
 (segment (start 196.1 112.315) (end 206 112.315) (width 0.4) (layer "B.Cu") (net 2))
 (segment (start 206 112.315) (end 207 113.315) (width 0.4) (layer "B.Cu") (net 2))
 (segment (start 183 118.895) (end 191.895 118.895) (width 0.4) (layer "B.Cu") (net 2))
 (segment (start 191.895 118.895) (end 192 119) (width 0.4) (layer "B.Cu") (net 2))
 (segment (start 192 119) (end 196.1 114.9) (width 0.4) (layer "B.Cu") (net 2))
 (segment (start 167 108.895) (end 167 114) (width 0.4) (layer "B.Cu") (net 2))
 (segment (start 183 116.355) (end 178.1 111.455) (width 0.4) (layer "B.Cu") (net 5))
 (segment (start 178.1 111.455) (end 178.1 110.315) (width 0.4) (layer "B.Cu") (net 5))
 (segment (start 231.1 101.315) (end 232.1 102.315) (width 1) (layer "B.Cu") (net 35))
 (segment (start 219.2 101.315) (end 231.1 101.315) (width 1) (layer "B.Cu") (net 35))
 (segment (start 232.02 107.315) (end 232.1 107.395) (width 1) (layer "F.Cu") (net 34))
 (segment (start 232.02 107.315) (end 232.1 107.395) (width 1) (layer "B.Cu") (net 34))
 (segment (start 205 107.315) (end 232.02 107.315) (width 1) (layer "B.Cu") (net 34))
 (segment (start 231.26 113.315) (end 232.1 112.475) (width 1) (layer "F.Cu") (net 33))
 (segment (start 231.26 113.315) (end 232.1 112.475) (width 1) (layer "B.Cu") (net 33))
 (segment (start 219.2 113.315) (end 231.26 113.315) (width 1) (layer "B.Cu") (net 33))
 (segment (start 234 46.175) (end 223.825 46.175) (width 0.4) (layer "B.Cu") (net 12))
 (segment (start 223.825 46.175) (end 201.84 68.16) (width 0.4) (layer "B.Cu") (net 12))
 (segment (start 201.84 68.16) (end 197 68.16) (width 0.4) (layer "B.Cu") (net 12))
 (segment (start 223 45) (end 212.54 45) (width 0.4) (layer "B.Cu") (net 9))
 (segment (start 212.54 45) (end 197 60.54) (width 0.4) (layer "B.Cu") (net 9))
 (segment (start 224.365 43.635) (end 223 45) (width 0.4) (layer "B.Cu") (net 9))
 (segment (start 234 43.635) (end 224.365 43.635) (width 0.4) (layer "B.Cu") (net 9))
 (segment (start 234 74.3575) (end 233.3575 75) (width 0.4) (layer "B.Cu") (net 24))
 (segment (start 233.3575 75) (end 223.18 75) (width 0.4) (layer "B.Cu") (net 24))
 (segment (start 223.18 75) (end 222.4 75.78) (width 0.4) (layer "B.Cu") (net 24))
 (segment (start 231.175 87.095) (end 222.4 78.32) (width 0.4) (layer "B.Cu") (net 23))
 (segment (start 234 87.095) (end 231.175 87.095) (width 0.4) (layer "B.Cu") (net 23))
 (segment (start 165.85 107.625) (end 157 98.775) (width 0.4) (layer "B.Cu") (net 3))
 (segment (start 157 98.775) (end 157 88) (width 0.4) (layer "B.Cu") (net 3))
 (segment (start 167 107.625) (end 165.85 107.625) (width 0.4) (layer "B.Cu") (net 3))
 (segment (start 157 88) (end 158 88) (width 0.4) (layer "B.Cu") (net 3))
 (segment (start 159 87) (end 180.84 87) (width 0.4) (layer "B.Cu") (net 3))
 (segment (start 158 88) (end 159 87) (width 0.4) (layer "B.Cu") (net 3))
 (segment (start 195.94 87) (end 197 85.94) (width 0.4) (layer "B.Cu") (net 19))
 (segment (start 191 87) (end 195.94 87) (width 0.4) (layer "B.Cu") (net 19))
 (segment (start 234 65) (end 225.56 65) (width 0.4) (layer "B.Cu") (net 27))
 (segment (start 225.56 65) (end 222.4 68.16) (width 0.4) (layer "B.Cu") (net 27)))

